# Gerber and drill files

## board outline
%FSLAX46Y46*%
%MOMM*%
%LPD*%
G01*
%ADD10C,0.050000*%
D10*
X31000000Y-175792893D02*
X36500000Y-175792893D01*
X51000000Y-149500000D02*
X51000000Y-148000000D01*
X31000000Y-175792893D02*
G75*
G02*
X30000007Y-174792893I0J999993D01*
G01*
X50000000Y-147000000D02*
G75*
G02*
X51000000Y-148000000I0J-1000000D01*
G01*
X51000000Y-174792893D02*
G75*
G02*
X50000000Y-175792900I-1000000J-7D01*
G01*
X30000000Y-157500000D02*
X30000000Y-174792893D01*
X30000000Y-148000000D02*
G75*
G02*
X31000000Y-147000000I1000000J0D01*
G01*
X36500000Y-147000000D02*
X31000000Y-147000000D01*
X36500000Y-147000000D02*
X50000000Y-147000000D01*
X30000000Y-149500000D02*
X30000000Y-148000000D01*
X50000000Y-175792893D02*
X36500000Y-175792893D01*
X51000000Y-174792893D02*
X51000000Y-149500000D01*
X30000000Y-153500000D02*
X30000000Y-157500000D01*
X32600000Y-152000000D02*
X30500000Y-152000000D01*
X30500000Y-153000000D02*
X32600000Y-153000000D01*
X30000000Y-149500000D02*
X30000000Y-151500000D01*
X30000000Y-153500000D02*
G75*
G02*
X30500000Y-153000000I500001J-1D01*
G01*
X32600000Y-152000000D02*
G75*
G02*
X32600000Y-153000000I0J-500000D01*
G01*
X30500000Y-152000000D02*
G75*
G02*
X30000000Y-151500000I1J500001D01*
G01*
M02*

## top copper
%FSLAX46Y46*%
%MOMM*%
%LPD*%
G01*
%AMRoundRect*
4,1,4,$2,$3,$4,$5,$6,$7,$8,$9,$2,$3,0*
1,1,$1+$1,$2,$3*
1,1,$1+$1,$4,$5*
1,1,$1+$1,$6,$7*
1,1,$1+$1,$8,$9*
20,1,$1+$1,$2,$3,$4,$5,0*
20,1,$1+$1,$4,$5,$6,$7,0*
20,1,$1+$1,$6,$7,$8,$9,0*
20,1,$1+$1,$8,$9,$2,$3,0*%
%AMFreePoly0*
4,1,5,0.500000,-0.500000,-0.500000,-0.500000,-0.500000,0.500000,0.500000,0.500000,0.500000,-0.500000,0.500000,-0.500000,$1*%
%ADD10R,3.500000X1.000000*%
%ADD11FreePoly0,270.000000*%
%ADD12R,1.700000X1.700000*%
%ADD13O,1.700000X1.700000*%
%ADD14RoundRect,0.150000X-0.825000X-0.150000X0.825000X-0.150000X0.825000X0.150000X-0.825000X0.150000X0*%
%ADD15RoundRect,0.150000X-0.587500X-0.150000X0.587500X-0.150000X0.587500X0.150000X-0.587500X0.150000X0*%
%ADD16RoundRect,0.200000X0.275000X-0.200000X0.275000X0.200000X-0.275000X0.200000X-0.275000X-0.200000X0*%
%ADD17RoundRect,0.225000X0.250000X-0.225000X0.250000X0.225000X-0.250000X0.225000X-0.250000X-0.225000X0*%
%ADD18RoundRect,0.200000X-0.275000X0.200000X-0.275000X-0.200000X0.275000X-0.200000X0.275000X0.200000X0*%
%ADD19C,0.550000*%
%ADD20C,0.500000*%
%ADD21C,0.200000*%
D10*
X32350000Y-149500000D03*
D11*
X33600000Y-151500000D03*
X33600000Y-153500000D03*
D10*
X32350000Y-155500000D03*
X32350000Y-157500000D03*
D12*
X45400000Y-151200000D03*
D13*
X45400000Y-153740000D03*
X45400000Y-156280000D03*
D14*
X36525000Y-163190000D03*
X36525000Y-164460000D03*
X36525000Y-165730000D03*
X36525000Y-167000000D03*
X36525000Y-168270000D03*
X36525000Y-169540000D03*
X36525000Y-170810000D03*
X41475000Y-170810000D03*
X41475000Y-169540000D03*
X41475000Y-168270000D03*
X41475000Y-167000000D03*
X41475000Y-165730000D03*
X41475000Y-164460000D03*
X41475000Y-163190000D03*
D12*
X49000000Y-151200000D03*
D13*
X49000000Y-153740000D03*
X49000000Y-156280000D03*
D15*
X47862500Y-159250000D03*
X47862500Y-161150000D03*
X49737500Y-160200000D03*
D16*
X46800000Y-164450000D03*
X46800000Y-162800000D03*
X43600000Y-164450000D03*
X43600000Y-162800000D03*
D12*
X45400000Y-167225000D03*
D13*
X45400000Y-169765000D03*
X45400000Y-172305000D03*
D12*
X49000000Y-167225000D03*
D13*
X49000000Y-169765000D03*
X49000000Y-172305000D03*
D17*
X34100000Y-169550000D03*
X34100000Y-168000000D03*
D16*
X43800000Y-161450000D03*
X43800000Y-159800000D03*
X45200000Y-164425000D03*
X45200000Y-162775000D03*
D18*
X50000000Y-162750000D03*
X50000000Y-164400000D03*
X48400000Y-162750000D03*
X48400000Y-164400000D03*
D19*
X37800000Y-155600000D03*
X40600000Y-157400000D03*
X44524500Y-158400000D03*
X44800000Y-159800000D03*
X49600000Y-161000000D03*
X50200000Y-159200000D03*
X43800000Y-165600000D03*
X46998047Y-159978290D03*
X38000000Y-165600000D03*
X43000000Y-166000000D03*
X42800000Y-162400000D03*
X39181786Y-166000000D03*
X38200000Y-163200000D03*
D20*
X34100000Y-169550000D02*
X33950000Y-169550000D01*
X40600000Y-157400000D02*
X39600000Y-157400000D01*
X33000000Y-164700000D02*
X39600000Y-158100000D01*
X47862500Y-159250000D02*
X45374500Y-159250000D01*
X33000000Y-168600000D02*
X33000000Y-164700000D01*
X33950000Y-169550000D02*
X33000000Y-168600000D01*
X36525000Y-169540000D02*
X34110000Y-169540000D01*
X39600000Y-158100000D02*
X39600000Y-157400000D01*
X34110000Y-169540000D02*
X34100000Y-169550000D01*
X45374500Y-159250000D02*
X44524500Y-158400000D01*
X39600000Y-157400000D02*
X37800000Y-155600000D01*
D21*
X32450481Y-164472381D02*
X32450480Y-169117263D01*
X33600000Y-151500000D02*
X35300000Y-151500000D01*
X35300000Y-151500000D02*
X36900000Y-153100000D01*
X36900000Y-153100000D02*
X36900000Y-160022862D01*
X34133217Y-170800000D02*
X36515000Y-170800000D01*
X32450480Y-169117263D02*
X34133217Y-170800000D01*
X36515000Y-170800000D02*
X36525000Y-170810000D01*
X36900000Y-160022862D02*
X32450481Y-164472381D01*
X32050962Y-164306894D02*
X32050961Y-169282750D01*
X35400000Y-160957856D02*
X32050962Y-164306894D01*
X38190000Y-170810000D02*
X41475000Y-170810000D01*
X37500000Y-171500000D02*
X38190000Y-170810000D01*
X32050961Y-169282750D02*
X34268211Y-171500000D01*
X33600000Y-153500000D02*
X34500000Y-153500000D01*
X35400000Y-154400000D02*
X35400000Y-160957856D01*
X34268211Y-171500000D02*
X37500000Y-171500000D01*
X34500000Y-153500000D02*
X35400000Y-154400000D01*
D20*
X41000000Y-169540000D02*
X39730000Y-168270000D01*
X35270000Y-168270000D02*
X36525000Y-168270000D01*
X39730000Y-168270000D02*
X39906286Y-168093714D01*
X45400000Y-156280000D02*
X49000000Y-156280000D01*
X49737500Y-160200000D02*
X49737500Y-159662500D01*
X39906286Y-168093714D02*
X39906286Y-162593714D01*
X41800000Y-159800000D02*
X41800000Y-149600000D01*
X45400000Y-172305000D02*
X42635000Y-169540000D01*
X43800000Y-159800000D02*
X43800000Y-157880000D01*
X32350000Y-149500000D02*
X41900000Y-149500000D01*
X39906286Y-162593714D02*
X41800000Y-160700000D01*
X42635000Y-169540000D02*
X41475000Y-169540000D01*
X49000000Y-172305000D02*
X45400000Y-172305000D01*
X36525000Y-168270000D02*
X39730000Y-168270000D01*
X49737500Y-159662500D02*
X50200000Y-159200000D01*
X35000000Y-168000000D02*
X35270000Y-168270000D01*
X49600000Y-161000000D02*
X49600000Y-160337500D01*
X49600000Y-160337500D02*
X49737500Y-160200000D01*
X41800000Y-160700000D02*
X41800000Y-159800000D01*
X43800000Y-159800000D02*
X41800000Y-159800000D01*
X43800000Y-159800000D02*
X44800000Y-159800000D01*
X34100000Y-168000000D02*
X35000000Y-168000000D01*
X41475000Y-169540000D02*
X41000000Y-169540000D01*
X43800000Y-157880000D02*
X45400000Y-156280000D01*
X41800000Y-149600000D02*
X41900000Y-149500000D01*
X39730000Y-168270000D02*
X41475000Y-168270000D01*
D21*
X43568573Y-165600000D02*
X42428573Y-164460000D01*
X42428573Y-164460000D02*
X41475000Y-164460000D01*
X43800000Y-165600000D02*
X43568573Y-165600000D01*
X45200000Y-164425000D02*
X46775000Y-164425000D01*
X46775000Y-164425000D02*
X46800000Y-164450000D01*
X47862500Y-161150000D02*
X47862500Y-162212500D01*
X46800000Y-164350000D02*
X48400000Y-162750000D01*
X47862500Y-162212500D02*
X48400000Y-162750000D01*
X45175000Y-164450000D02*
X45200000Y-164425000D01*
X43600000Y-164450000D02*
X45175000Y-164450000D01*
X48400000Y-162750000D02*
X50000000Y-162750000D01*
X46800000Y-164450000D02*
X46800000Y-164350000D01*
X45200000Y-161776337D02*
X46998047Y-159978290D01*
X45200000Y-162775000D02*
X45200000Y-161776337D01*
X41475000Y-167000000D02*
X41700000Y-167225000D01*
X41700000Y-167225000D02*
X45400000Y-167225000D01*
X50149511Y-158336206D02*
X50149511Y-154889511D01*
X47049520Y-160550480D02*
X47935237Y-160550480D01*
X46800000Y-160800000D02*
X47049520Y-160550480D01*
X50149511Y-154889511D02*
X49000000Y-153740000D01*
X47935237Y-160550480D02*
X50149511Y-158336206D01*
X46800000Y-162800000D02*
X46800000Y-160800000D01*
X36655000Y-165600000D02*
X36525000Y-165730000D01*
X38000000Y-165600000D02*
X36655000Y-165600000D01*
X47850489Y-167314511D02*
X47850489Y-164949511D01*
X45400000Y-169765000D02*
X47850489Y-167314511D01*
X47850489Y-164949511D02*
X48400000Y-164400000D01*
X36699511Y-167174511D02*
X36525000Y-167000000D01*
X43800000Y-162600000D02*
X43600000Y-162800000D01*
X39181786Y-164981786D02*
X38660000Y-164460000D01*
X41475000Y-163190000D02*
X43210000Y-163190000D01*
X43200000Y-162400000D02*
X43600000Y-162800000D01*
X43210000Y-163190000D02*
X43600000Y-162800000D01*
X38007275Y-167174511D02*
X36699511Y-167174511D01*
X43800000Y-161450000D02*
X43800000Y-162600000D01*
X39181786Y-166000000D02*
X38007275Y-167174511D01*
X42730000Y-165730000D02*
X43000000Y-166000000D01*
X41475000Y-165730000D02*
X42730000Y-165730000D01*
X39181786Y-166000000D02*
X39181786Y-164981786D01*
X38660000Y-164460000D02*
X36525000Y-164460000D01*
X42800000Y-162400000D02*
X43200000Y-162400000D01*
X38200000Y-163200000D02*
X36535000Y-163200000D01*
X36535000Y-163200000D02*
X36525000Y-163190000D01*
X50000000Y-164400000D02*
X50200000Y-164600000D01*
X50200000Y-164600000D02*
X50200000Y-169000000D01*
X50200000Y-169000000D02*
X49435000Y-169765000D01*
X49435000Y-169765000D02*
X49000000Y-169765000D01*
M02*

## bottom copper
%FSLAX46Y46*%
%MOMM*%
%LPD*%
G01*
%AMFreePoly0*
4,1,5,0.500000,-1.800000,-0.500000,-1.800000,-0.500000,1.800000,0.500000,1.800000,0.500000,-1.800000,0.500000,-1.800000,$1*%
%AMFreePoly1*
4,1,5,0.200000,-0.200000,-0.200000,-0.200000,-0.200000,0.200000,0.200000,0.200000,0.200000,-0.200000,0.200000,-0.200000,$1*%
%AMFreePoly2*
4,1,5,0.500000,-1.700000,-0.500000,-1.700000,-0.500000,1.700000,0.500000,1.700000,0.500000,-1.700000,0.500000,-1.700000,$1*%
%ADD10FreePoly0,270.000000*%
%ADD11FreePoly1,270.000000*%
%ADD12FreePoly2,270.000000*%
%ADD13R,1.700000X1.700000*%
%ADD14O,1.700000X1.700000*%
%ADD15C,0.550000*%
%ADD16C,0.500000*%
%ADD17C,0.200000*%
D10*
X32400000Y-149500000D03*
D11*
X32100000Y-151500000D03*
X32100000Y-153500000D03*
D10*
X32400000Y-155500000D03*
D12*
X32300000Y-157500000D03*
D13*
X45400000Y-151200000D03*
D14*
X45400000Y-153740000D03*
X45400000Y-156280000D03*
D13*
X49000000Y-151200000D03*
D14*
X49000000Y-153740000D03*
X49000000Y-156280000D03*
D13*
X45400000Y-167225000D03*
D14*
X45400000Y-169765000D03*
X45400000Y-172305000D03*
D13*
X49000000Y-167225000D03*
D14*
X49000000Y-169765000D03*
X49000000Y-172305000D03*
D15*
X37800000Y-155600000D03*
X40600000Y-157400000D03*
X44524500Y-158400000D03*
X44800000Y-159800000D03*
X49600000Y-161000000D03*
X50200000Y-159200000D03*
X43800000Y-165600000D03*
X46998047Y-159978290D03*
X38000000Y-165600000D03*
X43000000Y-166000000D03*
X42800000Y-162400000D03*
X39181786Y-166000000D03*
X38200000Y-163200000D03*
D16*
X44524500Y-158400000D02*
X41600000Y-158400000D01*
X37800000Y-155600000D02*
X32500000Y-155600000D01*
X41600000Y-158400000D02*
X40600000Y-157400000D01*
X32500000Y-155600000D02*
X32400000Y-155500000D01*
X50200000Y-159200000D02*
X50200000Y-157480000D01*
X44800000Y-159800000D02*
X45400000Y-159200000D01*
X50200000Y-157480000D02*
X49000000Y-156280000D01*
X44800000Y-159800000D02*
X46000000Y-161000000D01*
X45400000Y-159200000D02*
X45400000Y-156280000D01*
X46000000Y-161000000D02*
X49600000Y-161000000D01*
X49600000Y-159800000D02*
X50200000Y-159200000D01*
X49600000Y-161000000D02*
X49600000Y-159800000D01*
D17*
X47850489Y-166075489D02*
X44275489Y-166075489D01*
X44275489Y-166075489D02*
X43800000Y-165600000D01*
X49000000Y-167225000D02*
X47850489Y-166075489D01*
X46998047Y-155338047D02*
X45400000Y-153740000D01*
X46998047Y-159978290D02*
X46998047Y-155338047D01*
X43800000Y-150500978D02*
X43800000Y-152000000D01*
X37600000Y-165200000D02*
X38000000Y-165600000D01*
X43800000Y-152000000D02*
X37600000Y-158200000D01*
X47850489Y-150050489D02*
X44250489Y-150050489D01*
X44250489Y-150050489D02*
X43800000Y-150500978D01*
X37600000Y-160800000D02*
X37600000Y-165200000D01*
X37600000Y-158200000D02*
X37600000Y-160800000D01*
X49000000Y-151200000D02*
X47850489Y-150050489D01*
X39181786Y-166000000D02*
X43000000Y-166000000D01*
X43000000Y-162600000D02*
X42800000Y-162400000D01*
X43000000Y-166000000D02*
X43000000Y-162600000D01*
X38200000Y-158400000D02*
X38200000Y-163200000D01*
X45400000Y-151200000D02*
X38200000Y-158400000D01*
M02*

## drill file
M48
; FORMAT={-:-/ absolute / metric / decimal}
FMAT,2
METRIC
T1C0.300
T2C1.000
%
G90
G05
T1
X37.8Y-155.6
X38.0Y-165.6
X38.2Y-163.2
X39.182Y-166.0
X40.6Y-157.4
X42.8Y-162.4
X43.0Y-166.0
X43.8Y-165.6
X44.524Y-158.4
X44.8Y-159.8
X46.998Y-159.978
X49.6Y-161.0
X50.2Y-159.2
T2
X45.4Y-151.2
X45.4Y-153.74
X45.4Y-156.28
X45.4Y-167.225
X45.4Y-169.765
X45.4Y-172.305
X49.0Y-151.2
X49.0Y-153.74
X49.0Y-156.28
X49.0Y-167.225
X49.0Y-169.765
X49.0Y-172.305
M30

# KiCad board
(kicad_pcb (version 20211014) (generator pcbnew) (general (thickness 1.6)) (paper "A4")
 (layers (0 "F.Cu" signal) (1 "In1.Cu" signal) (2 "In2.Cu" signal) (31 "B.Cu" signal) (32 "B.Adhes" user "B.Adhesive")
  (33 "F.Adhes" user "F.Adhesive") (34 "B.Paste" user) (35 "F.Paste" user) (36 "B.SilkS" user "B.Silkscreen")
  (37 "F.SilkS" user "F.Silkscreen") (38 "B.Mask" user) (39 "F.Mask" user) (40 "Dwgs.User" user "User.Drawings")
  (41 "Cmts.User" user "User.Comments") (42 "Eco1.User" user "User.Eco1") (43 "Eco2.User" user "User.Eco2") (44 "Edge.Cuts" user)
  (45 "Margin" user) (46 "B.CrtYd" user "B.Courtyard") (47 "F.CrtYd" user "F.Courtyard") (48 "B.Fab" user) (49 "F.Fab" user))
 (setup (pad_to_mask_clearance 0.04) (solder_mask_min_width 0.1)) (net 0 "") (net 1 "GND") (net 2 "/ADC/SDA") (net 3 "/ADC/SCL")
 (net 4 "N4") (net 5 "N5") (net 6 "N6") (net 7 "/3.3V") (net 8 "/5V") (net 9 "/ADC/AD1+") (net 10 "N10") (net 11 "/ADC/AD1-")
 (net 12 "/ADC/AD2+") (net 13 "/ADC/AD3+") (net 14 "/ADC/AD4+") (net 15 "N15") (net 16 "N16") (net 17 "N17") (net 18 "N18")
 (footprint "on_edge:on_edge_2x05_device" (layer "F.Cu") (at 30 153.5 -90)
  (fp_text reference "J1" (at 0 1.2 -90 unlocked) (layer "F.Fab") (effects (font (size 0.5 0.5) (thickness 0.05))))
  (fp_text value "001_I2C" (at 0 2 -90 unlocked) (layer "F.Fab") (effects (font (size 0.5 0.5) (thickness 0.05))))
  (fp_line (start 0 0) (end 4 0) (layer "Edge.Cuts") (width 0.05))
  (fp_line (start -1.5 -2.6) (end -1.5 -0.5) (layer "Edge.Cuts") (width 0.05))
  (fp_line (start -0.5 -0.5) (end -0.5 -2.6) (layer "Edge.Cuts") (width 0.05))
  (fp_line (start -4 0) (end -2 0) (layer "Edge.Cuts") (width 0.05))
  (fp_arc (start 0 0) (mid -0.353553 -0.146447) (end -0.5 -0.5) (layer "Edge.Cuts") (width 0.05))
  (fp_arc (start -1.5 -2.6) (mid -1 -3.1) (end -0.5 -2.6) (layer "Edge.Cuts") (width 0.05))
  (fp_arc (start -1.5 -0.5) (mid -1.646447 -0.146447) (end -2 0) (layer "Edge.Cuts") (width 0.05))
  (pad "1" smd rect locked (at -4 -2.35 90) (size 1 3.5) (layers "F.Cu" "F.Mask") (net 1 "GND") (zone_connect 0))
  (pad "2" smd custom locked (at -2 -3.6 270) (size 1 1) (layers "F.Cu" "F.Mask") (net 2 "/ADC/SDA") (zone_connect 0)
   (options (clearance outline) (anchor rect)) (primitives))
  (pad "3" smd custom locked (at 0 -3.6 270) (size 1 1) (layers "F.Cu" "F.Mask") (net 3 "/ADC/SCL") (zone_connect 0)
   (options (clearance outline) (anchor rect)) (primitives))
  (pad "4" smd rect locked (at 2 -2.35 90) (size 1 3.5) (layers "F.Cu" "F.Mask") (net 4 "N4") (zone_connect 0))
  (pad "5" smd rect locked (at 4 -2.35 90) (size 1 3.5) (layers "F.Cu" "F.Mask") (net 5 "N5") (zone_connect 0))
  (pad "6" smd custom locked (at -4 -2.4 270) (size 1 3.6) (layers "B.Cu" "B.Mask") (zone_connect 0)
   (options (clearance outline) (anchor rect)) (primitives))
  (pad "7" smd custom locked (at -2 -2.1 270) (size 0.4 0.4) (layers "B.Cu" "B.Mask") (zone_connect 0)
   (options (clearance outline) (anchor rect)) (primitives))
  (pad "8" smd custom locked (at 0 -2.1 270) (size 0.4 0.4) (layers "B.Cu" "B.Mask") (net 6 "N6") (zone_connect 0)
   (options (clearance outline) (anchor rect)) (primitives))
  (pad "9" smd custom locked (at 2 -2.4 270) (size 1 3.6) (layers "B.Cu" "B.Mask") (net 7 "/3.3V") (zone_connect 0)
   (options (clearance outline) (anchor rect)) (primitives))
  (pad "10" smd custom locked (at 4 -2.3 270) (size 1 3.4) (layers "B.Cu" "B.Mask") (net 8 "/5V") (zone_connect 0)
   (options (clearance outline) (anchor rect)) (primitives)))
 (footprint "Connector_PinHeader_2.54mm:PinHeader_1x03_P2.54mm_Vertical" (layer "F.Cu") (at 45.4 151.2)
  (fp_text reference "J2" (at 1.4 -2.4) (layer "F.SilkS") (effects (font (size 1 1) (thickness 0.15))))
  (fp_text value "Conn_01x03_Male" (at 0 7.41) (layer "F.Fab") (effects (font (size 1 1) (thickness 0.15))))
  (pad "1" thru_hole rect locked (at 0 0) (size 1.7 1.7) (drill 1) (layers *.Cu *.Mask) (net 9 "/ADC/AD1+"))
  (pad "2" thru_hole oval locked (at 0 2.54) (size 1.7 1.7) (drill 1) (layers *.Cu *.Mask) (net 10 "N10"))
  (pad "3" thru_hole oval locked (at 0 5.08) (size 1.7 1.7) (drill 1) (layers *.Cu *.Mask) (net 1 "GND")))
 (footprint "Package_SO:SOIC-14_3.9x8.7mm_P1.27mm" (layer "F.Cu") (at 39 167)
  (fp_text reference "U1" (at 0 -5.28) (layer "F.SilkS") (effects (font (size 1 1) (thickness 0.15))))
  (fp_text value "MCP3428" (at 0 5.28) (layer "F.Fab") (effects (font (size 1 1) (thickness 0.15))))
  (pad "1" smd roundrect locked (at -2.475 -3.81) (size 1.95 0.6) (layers "F.Cu" "F.Paste" "F.Mask") (roundrect_rratio 0.25)
   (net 9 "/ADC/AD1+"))
  (pad "2" smd roundrect locked (at -2.475 -2.54) (size 1.95 0.6) (layers "F.Cu" "F.Paste" "F.Mask") (roundrect_rratio 0.25)
   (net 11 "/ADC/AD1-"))
  (pad "3" smd roundrect locked (at -2.475 -1.27) (size 1.95 0.6) (layers "F.Cu" "F.Paste" "F.Mask") (roundrect_rratio 0.25)
   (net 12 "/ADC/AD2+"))
  (pad "4" smd roundrect locked (at -2.475 0) (size 1.95 0.6) (layers "F.Cu" "F.Paste" "F.Mask") (roundrect_rratio 0.25)
   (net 11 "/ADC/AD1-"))
  (pad "5" smd roundrect locked (at -2.475 1.27) (size 1.95 0.6) (layers "F.Cu" "F.Paste" "F.Mask") (roundrect_rratio 0.25) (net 1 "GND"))
  (pad "6" smd roundrect locked (at -2.475 2.54) (size 1.95 0.6) (layers "F.Cu" "F.Paste" "F.Mask") (roundrect_rratio 0.25) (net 7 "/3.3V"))
  (pad "7" smd roundrect locked (at -2.475 3.81) (size 1.95 0.6) (layers "F.Cu" "F.Paste" "F.Mask") (roundrect_rratio 0.25)
   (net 2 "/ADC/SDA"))
  (pad "8" smd roundrect locked (at 2.475 3.81) (size 1.95 0.6) (layers "F.Cu" "F.Paste" "F.Mask") (roundrect_rratio 0.25)
   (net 3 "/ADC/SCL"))
  (pad "9" smd roundrect locked (at 2.475 2.54) (size 1.95 0.6) (layers "F.Cu" "F.Paste" "F.Mask") (roundrect_rratio 0.25) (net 1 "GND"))
  (pad "10" smd roundrect locked (at 2.475 1.27) (size 1.95 0.6) (layers "F.Cu" "F.Paste" "F.Mask") (roundrect_rratio 0.25) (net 1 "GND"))
  (pad "11" smd roundrect locked (at 2.475 0) (size 1.95 0.6) (layers "F.Cu" "F.Paste" "F.Mask") (roundrect_rratio 0.25)
   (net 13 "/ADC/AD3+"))
  (pad "12" smd roundrect locked (at 2.475 -1.27) (size 1.95 0.6) (layers "F.Cu" "F.Paste" "F.Mask") (roundrect_rratio 0.25)
   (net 11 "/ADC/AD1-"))
  (pad "13" smd roundrect locked (at 2.475 -2.54) (size 1.95 0.6) (layers "F.Cu" "F.Paste" "F.Mask") (roundrect_rratio 0.25)
   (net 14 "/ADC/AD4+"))
  (pad "14" smd roundrect locked (at 2.475 -3.81) (size 1.95 0.6) (layers "F.Cu" "F.Paste" "F.Mask") (roundrect_rratio 0.25)
   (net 11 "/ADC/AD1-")))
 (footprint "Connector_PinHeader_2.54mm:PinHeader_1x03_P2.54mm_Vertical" (layer "F.Cu") (at 49 151.2)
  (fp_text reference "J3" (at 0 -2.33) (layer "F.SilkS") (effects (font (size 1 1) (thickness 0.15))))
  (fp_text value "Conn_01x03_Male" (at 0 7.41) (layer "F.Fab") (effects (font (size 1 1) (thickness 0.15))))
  (pad "1" thru_hole rect locked (at 0 0) (size 1.7 1.7) (drill 1) (layers *.Cu *.Mask) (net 12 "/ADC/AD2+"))
  (pad "2" thru_hole oval locked (at 0 2.54) (size 1.7 1.7) (drill 1) (layers *.Cu *.Mask) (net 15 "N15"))
  (pad "3" thru_hole oval locked (at 0 5.08) (size 1.7 1.7) (drill 1) (layers *.Cu *.Mask) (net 1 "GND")))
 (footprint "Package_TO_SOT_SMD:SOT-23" (layer "F.Cu") (at 48.8 160.2)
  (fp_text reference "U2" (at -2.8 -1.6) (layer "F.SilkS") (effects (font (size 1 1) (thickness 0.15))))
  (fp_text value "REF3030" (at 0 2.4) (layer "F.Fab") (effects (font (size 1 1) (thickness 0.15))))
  (pad "1" smd roundrect locked (at -0.9375 -0.95) (size 1.475 0.6) (layers "F.Cu" "F.Paste" "F.Mask") (roundrect_rratio 0.25)
   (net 7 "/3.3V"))
  (pad "2" smd roundrect locked (at -0.9375 0.95) (size 1.475 0.6) (layers "F.Cu" "F.Paste" "F.Mask") (roundrect_rratio 0.25) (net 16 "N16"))
  (pad "3" smd roundrect locked (at 0.9375 0) (size 1.475 0.6) (layers "F.Cu" "F.Paste" "F.Mask") (roundrect_rratio 0.25) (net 1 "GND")))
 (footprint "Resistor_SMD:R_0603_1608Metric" (layer "F.Cu") (at 46.8 163.625 90)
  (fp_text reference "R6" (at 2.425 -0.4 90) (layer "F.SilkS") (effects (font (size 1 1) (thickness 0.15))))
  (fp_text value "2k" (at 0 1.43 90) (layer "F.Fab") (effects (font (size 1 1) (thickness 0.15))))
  (pad "1" smd roundrect locked (at -0.825 0 90) (size 0.8 0.95) (layers "F.Cu" "F.Paste" "F.Mask") (roundrect_rratio 0.25) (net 16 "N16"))
  (pad "2" smd roundrect locked (at 0.825 0 90) (size 0.8 0.95) (layers "F.Cu" "F.Paste" "F.Mask") (roundrect_rratio 0.25) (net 15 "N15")))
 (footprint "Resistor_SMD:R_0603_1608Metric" (layer "F.Cu") (at 43.6 163.625 90)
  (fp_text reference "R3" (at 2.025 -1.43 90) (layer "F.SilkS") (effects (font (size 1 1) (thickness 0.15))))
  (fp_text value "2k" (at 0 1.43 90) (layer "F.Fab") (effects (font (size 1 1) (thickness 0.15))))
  (pad "1" smd roundrect locked (at -0.825 0 90) (size 0.8 0.95) (layers "F.Cu" "F.Paste" "F.Mask") (roundrect_rratio 0.25) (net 16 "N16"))
  (pad "2" smd roundrect locked (at 0.825 0 90) (size 0.8 0.95) (layers "F.Cu" "F.Paste" "F.Mask") (roundrect_rratio 0.25)
   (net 11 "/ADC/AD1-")))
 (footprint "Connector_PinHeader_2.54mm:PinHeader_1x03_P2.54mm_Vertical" (layer "F.Cu") (at 45.4 167.225)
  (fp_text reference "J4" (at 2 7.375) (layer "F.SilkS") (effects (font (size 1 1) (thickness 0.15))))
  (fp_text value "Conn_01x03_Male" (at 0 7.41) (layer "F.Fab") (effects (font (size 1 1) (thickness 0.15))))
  (pad "1" thru_hole rect locked (at 0 0) (size 1.7 1.7) (drill 1) (layers *.Cu *.Mask) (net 13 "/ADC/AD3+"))
  (pad "2" thru_hole oval locked (at 0 2.54) (size 1.7 1.7) (drill 1) (layers *.Cu *.Mask) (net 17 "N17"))
  (pad "3" thru_hole oval locked (at 0 5.08) (size 1.7 1.7) (drill 1) (layers *.Cu *.Mask) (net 1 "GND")))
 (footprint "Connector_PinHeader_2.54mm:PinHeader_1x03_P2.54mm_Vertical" (layer "F.Cu") (at 49 167.225)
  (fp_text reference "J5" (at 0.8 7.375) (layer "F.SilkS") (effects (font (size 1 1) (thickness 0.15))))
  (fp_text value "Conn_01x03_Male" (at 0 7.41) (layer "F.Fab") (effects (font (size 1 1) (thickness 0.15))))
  (pad "1" thru_hole rect locked (at 0 0) (size 1.7 1.7) (drill 1) (layers *.Cu *.Mask) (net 14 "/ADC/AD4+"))
  (pad "2" thru_hole oval locked (at 0 2.54) (size 1.7 1.7) (drill 1) (layers *.Cu *.Mask) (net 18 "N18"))
  (pad "3" thru_hole oval locked (at 0 5.08) (size 1.7 1.7) (drill 1) (layers *.Cu *.Mask) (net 1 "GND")))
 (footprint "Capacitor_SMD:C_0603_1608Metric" (layer "F.Cu") (at 34.1 168.775 90)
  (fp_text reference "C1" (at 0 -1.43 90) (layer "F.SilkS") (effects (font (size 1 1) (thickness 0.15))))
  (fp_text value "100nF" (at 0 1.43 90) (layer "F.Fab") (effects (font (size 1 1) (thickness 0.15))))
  (pad "1" smd roundrect locked (at -0.775 0 90) (size 0.9 0.95) (layers "F.Cu" "F.Paste" "F.Mask") (roundrect_rratio 0.25) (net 7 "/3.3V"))
  (pad "2" smd roundrect locked (at 0.775 0 90) (size 0.9 0.95) (layers "F.Cu" "F.Paste" "F.Mask") (roundrect_rratio 0.25) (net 1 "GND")))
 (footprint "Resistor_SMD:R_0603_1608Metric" (layer "F.Cu") (at 43.8 160.625 90)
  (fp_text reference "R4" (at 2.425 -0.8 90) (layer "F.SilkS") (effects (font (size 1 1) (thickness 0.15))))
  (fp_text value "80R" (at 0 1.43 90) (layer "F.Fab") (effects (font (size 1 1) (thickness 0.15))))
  (pad "1" smd roundrect locked (at -0.825 0 90) (size 0.8 0.95) (layers "F.Cu" "F.Paste" "F.Mask") (roundrect_rratio 0.25)
   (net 11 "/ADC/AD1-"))
  (pad "2" smd roundrect locked (at 0.825 0 90) (size 0.8 0.95) (layers "F.Cu" "F.Paste" "F.Mask") (roundrect_rratio 0.25) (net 1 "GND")))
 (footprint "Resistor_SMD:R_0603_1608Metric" (layer "F.Cu") (at 45.2 163.6 90)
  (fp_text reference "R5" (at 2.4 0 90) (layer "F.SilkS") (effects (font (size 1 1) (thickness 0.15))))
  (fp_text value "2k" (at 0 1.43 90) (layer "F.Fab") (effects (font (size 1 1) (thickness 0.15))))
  (pad "1" smd roundrect locked (at -0.825 0 90) (size 0.8 0.95) (layers "F.Cu" "F.Paste" "F.Mask") (roundrect_rratio 0.25) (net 16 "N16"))
  (pad "2" smd roundrect locked (at 0.825 0 90) (size 0.8 0.95) (layers "F.Cu" "F.Paste" "F.Mask") (roundrect_rratio 0.25) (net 10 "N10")))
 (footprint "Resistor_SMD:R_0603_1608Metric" (layer "F.Cu") (at 50 163.575 -90)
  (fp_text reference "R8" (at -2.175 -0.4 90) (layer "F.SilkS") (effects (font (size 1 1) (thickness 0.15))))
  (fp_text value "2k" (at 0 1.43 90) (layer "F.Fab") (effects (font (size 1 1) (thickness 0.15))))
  (pad "1" smd roundrect locked (at -0.825 0 270) (size 0.8 0.95) (layers "F.Cu" "F.Paste" "F.Mask") (roundrect_rratio 0.25) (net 16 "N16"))
  (pad "2" smd roundrect locked (at 0.825 0 270) (size 0.8 0.95) (layers "F.Cu" "F.Paste" "F.Mask") (roundrect_rratio 0.25) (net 18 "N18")))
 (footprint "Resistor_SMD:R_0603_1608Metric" (layer "F.Cu") (at 48.4 163.575 -90)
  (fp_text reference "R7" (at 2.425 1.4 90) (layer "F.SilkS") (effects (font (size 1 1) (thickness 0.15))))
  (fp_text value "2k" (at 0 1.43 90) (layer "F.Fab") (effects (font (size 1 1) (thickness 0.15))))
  (pad "1" smd roundrect locked (at -0.825 0 270) (size 0.8 0.95) (layers "F.Cu" "F.Paste" "F.Mask") (roundrect_rratio 0.25) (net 16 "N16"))
  (pad "2" smd roundrect locked (at 0.825 0 270) (size 0.8 0.95) (layers "F.Cu" "F.Paste" "F.Mask") (roundrect_rratio 0.25) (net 17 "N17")))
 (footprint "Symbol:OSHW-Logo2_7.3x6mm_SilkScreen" (layer "B.Cu") (at 40.4 172.892893 180)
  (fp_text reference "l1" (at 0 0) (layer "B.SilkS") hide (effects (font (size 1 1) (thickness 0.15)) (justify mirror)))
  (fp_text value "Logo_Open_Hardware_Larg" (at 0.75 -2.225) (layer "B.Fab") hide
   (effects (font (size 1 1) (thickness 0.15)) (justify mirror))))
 (gr_line (start 31 175.792893) (end 36.5 175.792893) (layer "Edge.Cuts") (width 0.05))
 (gr_line (start 51 149.5) (end 51 148) (layer "Edge.Cuts") (width 0.05))
 (gr_arc (start 31 175.792893) (mid 30.292893 175.5) (end 30 174.792893) (layer "Edge.Cuts") (width 0.05))
 (gr_arc (start 50 147) (mid 50.707107 147.292893) (end 51 148) (layer "Edge.Cuts") (width 0.05))
 (gr_arc (start 51 174.792893) (mid 50.707107 175.5) (end 50 175.792893) (layer "Edge.Cuts") (width 0.05))
 (gr_line (start 30 157.5) (end 30 174.792893) (layer "Edge.Cuts") (width 0.05))
 (gr_arc (start 30 148) (mid 30.292893 147.292893) (end 31 147) (layer "Edge.Cuts") (width 0.05))
 (gr_line (start 36.5 147) (end 31 147) (layer "Edge.Cuts") (width 0.05))
 (gr_line (start 36.5 147) (end 50 147) (layer "Edge.Cuts") (width 0.05))
 (gr_line (start 30 149.5) (end 30 148) (layer "Edge.Cuts") (width 0.05))
 (gr_line (start 50 175.792893) (end 36.5 175.792893) (layer "Edge.Cuts") (width 0.05))
 (gr_line (start 51 174.792893) (end 51 149.5) (layer "Edge.Cuts") (width 0.05))
 (segment (start 34.1 169.55) (end 33.95 169.55) (width 0.5) (layer "F.Cu") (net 7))
 (segment (start 40.6 157.4) (end 39.6 157.4) (width 0.5) (layer "F.Cu") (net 7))
 (segment (start 33 164.7) (end 39.6 158.1) (width 0.5) (layer "F.Cu") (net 7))
 (segment (start 47.8625 159.25) (end 45.3745 159.25) (width 0.5) (layer "F.Cu") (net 7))
 (segment (start 33 168.6) (end 33 164.7) (width 0.5) (layer "F.Cu") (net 7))
 (segment (start 33.95 169.55) (end 33 168.6) (width 0.5) (layer "F.Cu") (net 7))
 (segment (start 36.525 169.54) (end 34.11 169.54) (width 0.5) (layer "F.Cu") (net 7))
 (segment (start 39.6 158.1) (end 39.6 157.4) (width 0.5) (layer "F.Cu") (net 7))
 (segment (start 34.11 169.54) (end 34.1 169.55) (width 0.5) (layer "F.Cu") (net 7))
 (segment (start 45.3745 159.25) (end 44.5245 158.4) (width 0.5) (layer "F.Cu") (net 7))
 (segment (start 39.6 157.4) (end 37.8 155.6) (width 0.5) (layer "F.Cu") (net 7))
 (via (at 37.8 155.6) (size 0.55) (drill 0.3) (layers "F.Cu" "B.Cu") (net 7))
 (via (at 40.6 157.4) (size 0.55) (drill 0.3) (layers "F.Cu" "B.Cu") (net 7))
 (via (at 44.5245 158.4) (size 0.55) (drill 0.3) (layers "F.Cu" "B.Cu") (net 7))
 (segment (start 44.5245 158.4) (end 41.6 158.4) (width 0.5) (layer "B.Cu") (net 7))
 (segment (start 37.8 155.6) (end 32.5 155.6) (width 0.5) (layer "B.Cu") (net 7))
 (segment (start 41.6 158.4) (end 40.6 157.4) (width 0.5) (layer "B.Cu") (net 7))
 (segment (start 32.5 155.6) (end 32.4 155.5) (width 0.5) (layer "B.Cu") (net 7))
 (segment (start 32.450481 164.472381) (end 32.45048 169.117263) (width 0.2) (layer "F.Cu") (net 2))
 (segment (start 33.6 151.5) (end 35.3 151.5) (width 0.2) (layer "F.Cu") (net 2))
 (segment (start 35.3 151.5) (end 36.9 153.1) (width 0.2) (layer "F.Cu") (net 2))
 (segment (start 36.9 153.1) (end 36.9 160.022862) (width 0.2) (layer "F.Cu") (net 2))
 (segment (start 34.133217 170.8) (end 36.515 170.8) (width 0.2) (layer "F.Cu") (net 2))
 (segment (start 32.45048 169.117263) (end 34.133217 170.8) (width 0.2) (layer "F.Cu") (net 2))
 (segment (start 36.515 170.8) (end 36.525 170.81) (width 0.2) (layer "F.Cu") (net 2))
 (segment (start 36.9 160.022862) (end 32.450481 164.472381) (width 0.2) (layer "F.Cu") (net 2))
 (segment (start 32.050962 164.306894) (end 32.050961 169.28275) (width 0.2) (layer "F.Cu") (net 3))
 (segment (start 35.4 160.957856) (end 32.050962 164.306894) (width 0.2) (layer "F.Cu") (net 3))
 (segment (start 38.19 170.81) (end 41.475 170.81) (width 0.2) (layer "F.Cu") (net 3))
 (segment (start 37.5 171.5) (end 38.19 170.81) (width 0.2) (layer "F.Cu") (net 3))
 (segment (start 32.050961 169.28275) (end 34.268211 171.5) (width 0.2) (layer "F.Cu") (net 3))
 (segment (start 33.6 153.5) (end 34.5 153.5) (width 0.2) (layer "F.Cu") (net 3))
 (segment (start 35.4 154.4) (end 35.4 160.957856) (width 0.2) (layer "F.Cu") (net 3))
 (segment (start 34.268211 171.5) (end 37.5 171.5) (width 0.2) (layer "F.Cu") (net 3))
 (segment (start 34.5 153.5) (end 35.4 154.4) (width 0.2) (layer "F.Cu") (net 3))
 (segment (start 41 169.54) (end 39.73 168.27) (width 0.5) (layer "F.Cu") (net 1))
 (segment (start 35.27 168.27) (end 36.525 168.27) (width 0.5) (layer "F.Cu") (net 1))
 (segment (start 39.73 168.27) (end 39.906286 168.093714) (width 0.5) (layer "F.Cu") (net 1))
 (segment (start 45.4 156.28) (end 49 156.28) (width 0.5) (layer "F.Cu") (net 1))
 (segment (start 49.7375 160.2) (end 49.7375 159.6625) (width 0.5) (layer "F.Cu") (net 1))
 (segment (start 39.906286 168.093714) (end 39.906286 162.593714) (width 0.5) (layer "F.Cu") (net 1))
 (segment (start 41.8 159.8) (end 41.8 149.6) (width 0.5) (layer "F.Cu") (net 1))
 (segment (start 45.4 172.305) (end 42.635 169.54) (width 0.5) (layer "F.Cu") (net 1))
 (segment (start 43.8 159.8) (end 43.8 157.88) (width 0.5) (layer "F.Cu") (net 1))
 (segment (start 32.35 149.5) (end 41.9 149.5) (width 0.5) (layer "F.Cu") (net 1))
 (segment (start 39.906286 162.593714) (end 41.8 160.7) (width 0.5) (layer "F.Cu") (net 1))
 (segment (start 42.635 169.54) (end 41.475 169.54) (width 0.5) (layer "F.Cu") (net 1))
 (segment (start 49 172.305) (end 45.4 172.305) (width 0.5) (layer "F.Cu") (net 1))
 (segment (start 36.525 168.27) (end 39.73 168.27) (width 0.5) (layer "F.Cu") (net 1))
 (segment (start 49.7375 159.6625) (end 50.2 159.2) (width 0.5) (layer "F.Cu") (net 1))
 (segment (start 35 168) (end 35.27 168.27) (width 0.5) (layer "F.Cu") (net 1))
 (segment (start 49.6 161) (end 49.6 160.3375) (width 0.5) (layer "F.Cu") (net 1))
 (segment (start 49.6 160.3375) (end 49.7375 160.2) (width 0.5) (layer "F.Cu") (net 1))
 (segment (start 41.8 160.7) (end 41.8 159.8) (width 0.5) (layer "F.Cu") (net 1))
 (segment (start 43.8 159.8) (end 41.8 159.8) (width 0.5) (layer "F.Cu") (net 1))
 (segment (start 43.8 159.8) (end 44.8 159.8) (width 0.5) (layer "F.Cu") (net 1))
 (segment (start 34.1 168) (end 35 168) (width 0.5) (layer "F.Cu") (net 1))
 (segment (start 41.475 169.54) (end 41 169.54) (width 0.5) (layer "F.Cu") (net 1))
 (segment (start 43.8 157.88) (end 45.4 156.28) (width 0.5) (layer "F.Cu") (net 1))
 (segment (start 41.8 149.6) (end 41.9 149.5) (width 0.5) (layer "F.Cu") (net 1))
 (segment (start 39.73 168.27) (end 41.475 168.27) (width 0.5) (layer "F.Cu") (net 1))
 (via (at 44.8 159.8) (size 0.55) (drill 0.3) (layers "F.Cu" "B.Cu") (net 1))
 (via (at 49.6 161) (size 0.55) (drill 0.3) (layers "F.Cu" "B.Cu") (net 1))
 (via (at 50.2 159.2) (size 0.55) (drill 0.3) (layers "F.Cu" "B.Cu") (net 1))
 (segment (start 50.2 159.2) (end 50.2 157.48) (width 0.5) (layer "B.Cu") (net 1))
 (segment (start 44.8 159.8) (end 45.4 159.2) (width 0.5) (layer "B.Cu") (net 1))
 (segment (start 50.2 157.48) (end 49 156.28) (width 0.5) (layer "B.Cu") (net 1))
 (segment (start 44.8 159.8) (end 46 161) (width 0.5) (layer "B.Cu") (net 1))
 (segment (start 45.4 159.2) (end 45.4 156.28) (width 0.5) (layer "B.Cu") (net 1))
 (segment (start 46 161) (end 49.6 161) (width 0.5) (layer "B.Cu") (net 1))
 (segment (start 49.6 159.8) (end 50.2 159.2) (width 0.5) (layer "B.Cu") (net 1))
 (segment (start 49.6 161) (end 49.6 159.8) (width 0.5) (layer "B.Cu") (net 1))
 (segment (start 43.568573 165.6) (end 42.428573 164.46) (width 0.2) (layer "F.Cu") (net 14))
 (segment (start 42.428573 164.46) (end 41.475 164.46) (width 0.2) (layer "F.Cu") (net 14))
 (segment (start 43.8 165.6) (end 43.568573 165.6) (width 0.2) (layer "F.Cu") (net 14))
 (via (at 43.8 165.6) (size 0.55) (drill 0.3) (layers "F.Cu" "B.Cu") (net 14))
 (segment (start 47.850489 166.075489) (end 44.275489 166.075489) (width 0.2) (layer "B.Cu") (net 14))
 (segment (start 44.275489 166.075489) (end 43.8 165.6) (width 0.2) (layer "B.Cu") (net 14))
 (segment (start 49 167.225) (end 47.850489 166.075489) (width 0.2) (layer "B.Cu") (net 14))
 (segment (start 45.2 164.425) (end 46.775 164.425) (width 0.2) (layer "F.Cu") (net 16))
 (segment (start 46.775 164.425) (end 46.8 164.45) (width 0.2) (layer "F.Cu") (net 16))
 (segment (start 47.8625 161.15) (end 47.8625 162.2125) (width 0.2) (layer "F.Cu") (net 16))
 (segment (start 46.8 164.35) (end 48.4 162.75) (width 0.2) (layer "F.Cu") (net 16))
 (segment (start 47.8625 162.2125) (end 48.4 162.75) (width 0.2) (layer "F.Cu") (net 16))
 (segment (start 45.175 164.45) (end 45.2 164.425) (width 0.2) (layer "F.Cu") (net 16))
 (segment (start 43.6 164.45) (end 45.175 164.45) (width 0.2) (layer "F.Cu") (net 16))
 (segment (start 48.4 162.75) (end 50 162.75) (width 0.2) (layer "F.Cu") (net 16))
 (segment (start 46.8 164.45) (end 46.8 164.35) (width 0.2) (layer "F.Cu") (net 16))
 (segment (start 45.2 161.776337) (end 46.998047 159.97829) (width 0.2) (layer "F.Cu") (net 10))
 (segment (start 45.2 162.775) (end 45.2 161.776337) (width 0.2) (layer "F.Cu") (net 10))
 (via (at 46.998047 159.97829) (size 0.55) (drill 0.3) (layers "F.Cu" "B.Cu") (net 10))
 (segment (start 46.998047 155.338047) (end 45.4 153.74) (width 0.2) (layer "B.Cu") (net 10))
 (segment (start 46.998047 159.97829) (end 46.998047 155.338047) (width 0.2) (layer "B.Cu") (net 10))
 (segment (start 41.475 167) (end 41.7 167.225) (width 0.2) (layer "F.Cu") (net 13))
 (segment (start 41.7 167.225) (end 45.4 167.225) (width 0.2) (layer "F.Cu") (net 13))
 (segment (start 50.149511 158.336206) (end 50.149511 154.889511) (width 0.2) (layer "F.Cu") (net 15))
 (segment (start 47.04952 160.55048) (end 47.935237 160.55048) (width 0.2) (layer "F.Cu") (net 15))
 (segment (start 46.8 160.8) (end 47.04952 160.55048) (width 0.2) (layer "F.Cu") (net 15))
 (segment (start 50.149511 154.889511) (end 49 153.74) (width 0.2) (layer "F.Cu") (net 15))
 (segment (start 47.935237 160.55048) (end 50.149511 158.336206) (width 0.2) (layer "F.Cu") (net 15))
 (segment (start 46.8 162.8) (end 46.8 160.8) (width 0.2) (layer "F.Cu") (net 15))
 (segment (start 36.655 165.6) (end 36.525 165.73) (width 0.2) (layer "F.Cu") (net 12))
 (segment (start 38 165.6) (end 36.655 165.6) (width 0.2) (layer "F.Cu") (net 12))
 (via (at 38 165.6) (size 0.55) (drill 0.3) (layers "F.Cu" "B.Cu") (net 12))
 (segment (start 43.8 150.500978) (end 43.8 152) (width 0.2) (layer "B.Cu") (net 12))
 (segment (start 37.6 165.2) (end 38 165.6) (width 0.2) (layer "B.Cu") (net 12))
 (segment (start 43.8 152) (end 37.6 158.2) (width 0.2) (layer "B.Cu") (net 12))
 (segment (start 47.850489 150.050489) (end 44.250489 150.050489) (width 0.2) (layer "B.Cu") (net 12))
 (segment (start 44.250489 150.050489) (end 43.8 150.500978) (width 0.2) (layer "B.Cu") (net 12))
 (segment (start 37.6 160.8) (end 37.6 165.2) (width 0.2) (layer "B.Cu") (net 12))
 (segment (start 37.6 158.2) (end 37.6 160.8) (width 0.2) (layer "B.Cu") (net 12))
 (segment (start 49 151.2) (end 47.850489 150.050489) (width 0.2) (layer "B.Cu") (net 12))
 (segment (start 47.850489 167.314511) (end 47.850489 164.949511) (width 0.2) (layer "F.Cu") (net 17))
 (segment (start 45.4 169.765) (end 47.850489 167.314511) (width 0.2) (layer "F.Cu") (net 17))
 (segment (start 47.850489 164.949511) (end 48.4 164.4) (width 0.2) (layer "F.Cu") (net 17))
 (segment (start 36.699511 167.174511) (end 36.525 167) (width 0.2) (layer "F.Cu") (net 11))
 (segment (start 43.8 162.6) (end 43.6 162.8) (width 0.2) (layer "F.Cu") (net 11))
 (segment (start 39.181786 164.981786) (end 38.66 164.46) (width 0.2) (layer "F.Cu") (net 11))
 (segment (start 41.475 163.19) (end 43.21 163.19) (width 0.2) (layer "F.Cu") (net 11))
 (segment (start 43.2 162.4) (end 43.6 162.8) (width 0.2) (layer "F.Cu") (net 11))
 (segment (start 43.21 163.19) (end 43.6 162.8) (width 0.2) (layer "F.Cu") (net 11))
 (segment (start 38.007275 167.174511) (end 36.699511 167.174511) (width 0.2) (layer "F.Cu") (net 11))
 (segment (start 43.8 161.45) (end 43.8 162.6) (width 0.2) (layer "F.Cu") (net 11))
 (segment (start 39.181786 166) (end 38.007275 167.174511) (width 0.2) (layer "F.Cu") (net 11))
 (segment (start 42.73 165.73) (end 43 166) (width 0.2) (layer "F.Cu") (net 11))
 (segment (start 41.475 165.73) (end 42.73 165.73) (width 0.2) (layer "F.Cu") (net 11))
 (segment (start 39.181786 166) (end 39.181786 164.981786) (width 0.2) (layer "F.Cu") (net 11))
 (segment (start 38.66 164.46) (end 36.525 164.46) (width 0.2) (layer "F.Cu") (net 11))
 (segment (start 42.8 162.4) (end 43.2 162.4) (width 0.2) (layer "F.Cu") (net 11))
 (via (at 43 166) (size 0.55) (drill 0.3) (layers "F.Cu" "B.Cu") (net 11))
 (via (at 42.8 162.4) (size 0.55) (drill 0.3) (layers "F.Cu" "B.Cu") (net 11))
 (via (at 39.181786 166) (size 0.55) (drill 0.3) (layers "F.Cu" "B.Cu") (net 11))
 (segment (start 39.181786 166) (end 43 166) (width 0.2) (layer "B.Cu") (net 11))
 (segment (start 43 162.6) (end 42.8 162.4) (width 0.2) (layer "B.Cu") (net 11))
 (segment (start 43 166) (end 43 162.6) (width 0.2) (layer "B.Cu") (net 11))
 (segment (start 38.2 163.2) (end 36.535 163.2) (width 0.2) (layer "F.Cu") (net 9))
 (segment (start 36.535 163.2) (end 36.525 163.19) (width 0.2) (layer "F.Cu") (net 9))
 (via (at 38.2 163.2) (size 0.55) (drill 0.3) (layers "F.Cu" "B.Cu") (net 9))
 (segment (start 38.2 158.4) (end 38.2 163.2) (width 0.2) (layer "B.Cu") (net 9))
 (segment (start 45.4 151.2) (end 38.2 158.4) (width 0.2) (layer "B.Cu") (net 9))
 (segment (start 50 164.4) (end 50.2 164.6) (width 0.2) (layer "F.Cu") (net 18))
 (segment (start 50.2 164.6) (end 50.2 169) (width 0.2) (layer "F.Cu") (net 18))
 (segment (start 50.2 169) (end 49.435 169.765) (width 0.2) (layer "F.Cu") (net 18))
 (segment (start 49.435 169.765) (end 49 169.765) (width 0.2) (layer "F.Cu") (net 18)))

